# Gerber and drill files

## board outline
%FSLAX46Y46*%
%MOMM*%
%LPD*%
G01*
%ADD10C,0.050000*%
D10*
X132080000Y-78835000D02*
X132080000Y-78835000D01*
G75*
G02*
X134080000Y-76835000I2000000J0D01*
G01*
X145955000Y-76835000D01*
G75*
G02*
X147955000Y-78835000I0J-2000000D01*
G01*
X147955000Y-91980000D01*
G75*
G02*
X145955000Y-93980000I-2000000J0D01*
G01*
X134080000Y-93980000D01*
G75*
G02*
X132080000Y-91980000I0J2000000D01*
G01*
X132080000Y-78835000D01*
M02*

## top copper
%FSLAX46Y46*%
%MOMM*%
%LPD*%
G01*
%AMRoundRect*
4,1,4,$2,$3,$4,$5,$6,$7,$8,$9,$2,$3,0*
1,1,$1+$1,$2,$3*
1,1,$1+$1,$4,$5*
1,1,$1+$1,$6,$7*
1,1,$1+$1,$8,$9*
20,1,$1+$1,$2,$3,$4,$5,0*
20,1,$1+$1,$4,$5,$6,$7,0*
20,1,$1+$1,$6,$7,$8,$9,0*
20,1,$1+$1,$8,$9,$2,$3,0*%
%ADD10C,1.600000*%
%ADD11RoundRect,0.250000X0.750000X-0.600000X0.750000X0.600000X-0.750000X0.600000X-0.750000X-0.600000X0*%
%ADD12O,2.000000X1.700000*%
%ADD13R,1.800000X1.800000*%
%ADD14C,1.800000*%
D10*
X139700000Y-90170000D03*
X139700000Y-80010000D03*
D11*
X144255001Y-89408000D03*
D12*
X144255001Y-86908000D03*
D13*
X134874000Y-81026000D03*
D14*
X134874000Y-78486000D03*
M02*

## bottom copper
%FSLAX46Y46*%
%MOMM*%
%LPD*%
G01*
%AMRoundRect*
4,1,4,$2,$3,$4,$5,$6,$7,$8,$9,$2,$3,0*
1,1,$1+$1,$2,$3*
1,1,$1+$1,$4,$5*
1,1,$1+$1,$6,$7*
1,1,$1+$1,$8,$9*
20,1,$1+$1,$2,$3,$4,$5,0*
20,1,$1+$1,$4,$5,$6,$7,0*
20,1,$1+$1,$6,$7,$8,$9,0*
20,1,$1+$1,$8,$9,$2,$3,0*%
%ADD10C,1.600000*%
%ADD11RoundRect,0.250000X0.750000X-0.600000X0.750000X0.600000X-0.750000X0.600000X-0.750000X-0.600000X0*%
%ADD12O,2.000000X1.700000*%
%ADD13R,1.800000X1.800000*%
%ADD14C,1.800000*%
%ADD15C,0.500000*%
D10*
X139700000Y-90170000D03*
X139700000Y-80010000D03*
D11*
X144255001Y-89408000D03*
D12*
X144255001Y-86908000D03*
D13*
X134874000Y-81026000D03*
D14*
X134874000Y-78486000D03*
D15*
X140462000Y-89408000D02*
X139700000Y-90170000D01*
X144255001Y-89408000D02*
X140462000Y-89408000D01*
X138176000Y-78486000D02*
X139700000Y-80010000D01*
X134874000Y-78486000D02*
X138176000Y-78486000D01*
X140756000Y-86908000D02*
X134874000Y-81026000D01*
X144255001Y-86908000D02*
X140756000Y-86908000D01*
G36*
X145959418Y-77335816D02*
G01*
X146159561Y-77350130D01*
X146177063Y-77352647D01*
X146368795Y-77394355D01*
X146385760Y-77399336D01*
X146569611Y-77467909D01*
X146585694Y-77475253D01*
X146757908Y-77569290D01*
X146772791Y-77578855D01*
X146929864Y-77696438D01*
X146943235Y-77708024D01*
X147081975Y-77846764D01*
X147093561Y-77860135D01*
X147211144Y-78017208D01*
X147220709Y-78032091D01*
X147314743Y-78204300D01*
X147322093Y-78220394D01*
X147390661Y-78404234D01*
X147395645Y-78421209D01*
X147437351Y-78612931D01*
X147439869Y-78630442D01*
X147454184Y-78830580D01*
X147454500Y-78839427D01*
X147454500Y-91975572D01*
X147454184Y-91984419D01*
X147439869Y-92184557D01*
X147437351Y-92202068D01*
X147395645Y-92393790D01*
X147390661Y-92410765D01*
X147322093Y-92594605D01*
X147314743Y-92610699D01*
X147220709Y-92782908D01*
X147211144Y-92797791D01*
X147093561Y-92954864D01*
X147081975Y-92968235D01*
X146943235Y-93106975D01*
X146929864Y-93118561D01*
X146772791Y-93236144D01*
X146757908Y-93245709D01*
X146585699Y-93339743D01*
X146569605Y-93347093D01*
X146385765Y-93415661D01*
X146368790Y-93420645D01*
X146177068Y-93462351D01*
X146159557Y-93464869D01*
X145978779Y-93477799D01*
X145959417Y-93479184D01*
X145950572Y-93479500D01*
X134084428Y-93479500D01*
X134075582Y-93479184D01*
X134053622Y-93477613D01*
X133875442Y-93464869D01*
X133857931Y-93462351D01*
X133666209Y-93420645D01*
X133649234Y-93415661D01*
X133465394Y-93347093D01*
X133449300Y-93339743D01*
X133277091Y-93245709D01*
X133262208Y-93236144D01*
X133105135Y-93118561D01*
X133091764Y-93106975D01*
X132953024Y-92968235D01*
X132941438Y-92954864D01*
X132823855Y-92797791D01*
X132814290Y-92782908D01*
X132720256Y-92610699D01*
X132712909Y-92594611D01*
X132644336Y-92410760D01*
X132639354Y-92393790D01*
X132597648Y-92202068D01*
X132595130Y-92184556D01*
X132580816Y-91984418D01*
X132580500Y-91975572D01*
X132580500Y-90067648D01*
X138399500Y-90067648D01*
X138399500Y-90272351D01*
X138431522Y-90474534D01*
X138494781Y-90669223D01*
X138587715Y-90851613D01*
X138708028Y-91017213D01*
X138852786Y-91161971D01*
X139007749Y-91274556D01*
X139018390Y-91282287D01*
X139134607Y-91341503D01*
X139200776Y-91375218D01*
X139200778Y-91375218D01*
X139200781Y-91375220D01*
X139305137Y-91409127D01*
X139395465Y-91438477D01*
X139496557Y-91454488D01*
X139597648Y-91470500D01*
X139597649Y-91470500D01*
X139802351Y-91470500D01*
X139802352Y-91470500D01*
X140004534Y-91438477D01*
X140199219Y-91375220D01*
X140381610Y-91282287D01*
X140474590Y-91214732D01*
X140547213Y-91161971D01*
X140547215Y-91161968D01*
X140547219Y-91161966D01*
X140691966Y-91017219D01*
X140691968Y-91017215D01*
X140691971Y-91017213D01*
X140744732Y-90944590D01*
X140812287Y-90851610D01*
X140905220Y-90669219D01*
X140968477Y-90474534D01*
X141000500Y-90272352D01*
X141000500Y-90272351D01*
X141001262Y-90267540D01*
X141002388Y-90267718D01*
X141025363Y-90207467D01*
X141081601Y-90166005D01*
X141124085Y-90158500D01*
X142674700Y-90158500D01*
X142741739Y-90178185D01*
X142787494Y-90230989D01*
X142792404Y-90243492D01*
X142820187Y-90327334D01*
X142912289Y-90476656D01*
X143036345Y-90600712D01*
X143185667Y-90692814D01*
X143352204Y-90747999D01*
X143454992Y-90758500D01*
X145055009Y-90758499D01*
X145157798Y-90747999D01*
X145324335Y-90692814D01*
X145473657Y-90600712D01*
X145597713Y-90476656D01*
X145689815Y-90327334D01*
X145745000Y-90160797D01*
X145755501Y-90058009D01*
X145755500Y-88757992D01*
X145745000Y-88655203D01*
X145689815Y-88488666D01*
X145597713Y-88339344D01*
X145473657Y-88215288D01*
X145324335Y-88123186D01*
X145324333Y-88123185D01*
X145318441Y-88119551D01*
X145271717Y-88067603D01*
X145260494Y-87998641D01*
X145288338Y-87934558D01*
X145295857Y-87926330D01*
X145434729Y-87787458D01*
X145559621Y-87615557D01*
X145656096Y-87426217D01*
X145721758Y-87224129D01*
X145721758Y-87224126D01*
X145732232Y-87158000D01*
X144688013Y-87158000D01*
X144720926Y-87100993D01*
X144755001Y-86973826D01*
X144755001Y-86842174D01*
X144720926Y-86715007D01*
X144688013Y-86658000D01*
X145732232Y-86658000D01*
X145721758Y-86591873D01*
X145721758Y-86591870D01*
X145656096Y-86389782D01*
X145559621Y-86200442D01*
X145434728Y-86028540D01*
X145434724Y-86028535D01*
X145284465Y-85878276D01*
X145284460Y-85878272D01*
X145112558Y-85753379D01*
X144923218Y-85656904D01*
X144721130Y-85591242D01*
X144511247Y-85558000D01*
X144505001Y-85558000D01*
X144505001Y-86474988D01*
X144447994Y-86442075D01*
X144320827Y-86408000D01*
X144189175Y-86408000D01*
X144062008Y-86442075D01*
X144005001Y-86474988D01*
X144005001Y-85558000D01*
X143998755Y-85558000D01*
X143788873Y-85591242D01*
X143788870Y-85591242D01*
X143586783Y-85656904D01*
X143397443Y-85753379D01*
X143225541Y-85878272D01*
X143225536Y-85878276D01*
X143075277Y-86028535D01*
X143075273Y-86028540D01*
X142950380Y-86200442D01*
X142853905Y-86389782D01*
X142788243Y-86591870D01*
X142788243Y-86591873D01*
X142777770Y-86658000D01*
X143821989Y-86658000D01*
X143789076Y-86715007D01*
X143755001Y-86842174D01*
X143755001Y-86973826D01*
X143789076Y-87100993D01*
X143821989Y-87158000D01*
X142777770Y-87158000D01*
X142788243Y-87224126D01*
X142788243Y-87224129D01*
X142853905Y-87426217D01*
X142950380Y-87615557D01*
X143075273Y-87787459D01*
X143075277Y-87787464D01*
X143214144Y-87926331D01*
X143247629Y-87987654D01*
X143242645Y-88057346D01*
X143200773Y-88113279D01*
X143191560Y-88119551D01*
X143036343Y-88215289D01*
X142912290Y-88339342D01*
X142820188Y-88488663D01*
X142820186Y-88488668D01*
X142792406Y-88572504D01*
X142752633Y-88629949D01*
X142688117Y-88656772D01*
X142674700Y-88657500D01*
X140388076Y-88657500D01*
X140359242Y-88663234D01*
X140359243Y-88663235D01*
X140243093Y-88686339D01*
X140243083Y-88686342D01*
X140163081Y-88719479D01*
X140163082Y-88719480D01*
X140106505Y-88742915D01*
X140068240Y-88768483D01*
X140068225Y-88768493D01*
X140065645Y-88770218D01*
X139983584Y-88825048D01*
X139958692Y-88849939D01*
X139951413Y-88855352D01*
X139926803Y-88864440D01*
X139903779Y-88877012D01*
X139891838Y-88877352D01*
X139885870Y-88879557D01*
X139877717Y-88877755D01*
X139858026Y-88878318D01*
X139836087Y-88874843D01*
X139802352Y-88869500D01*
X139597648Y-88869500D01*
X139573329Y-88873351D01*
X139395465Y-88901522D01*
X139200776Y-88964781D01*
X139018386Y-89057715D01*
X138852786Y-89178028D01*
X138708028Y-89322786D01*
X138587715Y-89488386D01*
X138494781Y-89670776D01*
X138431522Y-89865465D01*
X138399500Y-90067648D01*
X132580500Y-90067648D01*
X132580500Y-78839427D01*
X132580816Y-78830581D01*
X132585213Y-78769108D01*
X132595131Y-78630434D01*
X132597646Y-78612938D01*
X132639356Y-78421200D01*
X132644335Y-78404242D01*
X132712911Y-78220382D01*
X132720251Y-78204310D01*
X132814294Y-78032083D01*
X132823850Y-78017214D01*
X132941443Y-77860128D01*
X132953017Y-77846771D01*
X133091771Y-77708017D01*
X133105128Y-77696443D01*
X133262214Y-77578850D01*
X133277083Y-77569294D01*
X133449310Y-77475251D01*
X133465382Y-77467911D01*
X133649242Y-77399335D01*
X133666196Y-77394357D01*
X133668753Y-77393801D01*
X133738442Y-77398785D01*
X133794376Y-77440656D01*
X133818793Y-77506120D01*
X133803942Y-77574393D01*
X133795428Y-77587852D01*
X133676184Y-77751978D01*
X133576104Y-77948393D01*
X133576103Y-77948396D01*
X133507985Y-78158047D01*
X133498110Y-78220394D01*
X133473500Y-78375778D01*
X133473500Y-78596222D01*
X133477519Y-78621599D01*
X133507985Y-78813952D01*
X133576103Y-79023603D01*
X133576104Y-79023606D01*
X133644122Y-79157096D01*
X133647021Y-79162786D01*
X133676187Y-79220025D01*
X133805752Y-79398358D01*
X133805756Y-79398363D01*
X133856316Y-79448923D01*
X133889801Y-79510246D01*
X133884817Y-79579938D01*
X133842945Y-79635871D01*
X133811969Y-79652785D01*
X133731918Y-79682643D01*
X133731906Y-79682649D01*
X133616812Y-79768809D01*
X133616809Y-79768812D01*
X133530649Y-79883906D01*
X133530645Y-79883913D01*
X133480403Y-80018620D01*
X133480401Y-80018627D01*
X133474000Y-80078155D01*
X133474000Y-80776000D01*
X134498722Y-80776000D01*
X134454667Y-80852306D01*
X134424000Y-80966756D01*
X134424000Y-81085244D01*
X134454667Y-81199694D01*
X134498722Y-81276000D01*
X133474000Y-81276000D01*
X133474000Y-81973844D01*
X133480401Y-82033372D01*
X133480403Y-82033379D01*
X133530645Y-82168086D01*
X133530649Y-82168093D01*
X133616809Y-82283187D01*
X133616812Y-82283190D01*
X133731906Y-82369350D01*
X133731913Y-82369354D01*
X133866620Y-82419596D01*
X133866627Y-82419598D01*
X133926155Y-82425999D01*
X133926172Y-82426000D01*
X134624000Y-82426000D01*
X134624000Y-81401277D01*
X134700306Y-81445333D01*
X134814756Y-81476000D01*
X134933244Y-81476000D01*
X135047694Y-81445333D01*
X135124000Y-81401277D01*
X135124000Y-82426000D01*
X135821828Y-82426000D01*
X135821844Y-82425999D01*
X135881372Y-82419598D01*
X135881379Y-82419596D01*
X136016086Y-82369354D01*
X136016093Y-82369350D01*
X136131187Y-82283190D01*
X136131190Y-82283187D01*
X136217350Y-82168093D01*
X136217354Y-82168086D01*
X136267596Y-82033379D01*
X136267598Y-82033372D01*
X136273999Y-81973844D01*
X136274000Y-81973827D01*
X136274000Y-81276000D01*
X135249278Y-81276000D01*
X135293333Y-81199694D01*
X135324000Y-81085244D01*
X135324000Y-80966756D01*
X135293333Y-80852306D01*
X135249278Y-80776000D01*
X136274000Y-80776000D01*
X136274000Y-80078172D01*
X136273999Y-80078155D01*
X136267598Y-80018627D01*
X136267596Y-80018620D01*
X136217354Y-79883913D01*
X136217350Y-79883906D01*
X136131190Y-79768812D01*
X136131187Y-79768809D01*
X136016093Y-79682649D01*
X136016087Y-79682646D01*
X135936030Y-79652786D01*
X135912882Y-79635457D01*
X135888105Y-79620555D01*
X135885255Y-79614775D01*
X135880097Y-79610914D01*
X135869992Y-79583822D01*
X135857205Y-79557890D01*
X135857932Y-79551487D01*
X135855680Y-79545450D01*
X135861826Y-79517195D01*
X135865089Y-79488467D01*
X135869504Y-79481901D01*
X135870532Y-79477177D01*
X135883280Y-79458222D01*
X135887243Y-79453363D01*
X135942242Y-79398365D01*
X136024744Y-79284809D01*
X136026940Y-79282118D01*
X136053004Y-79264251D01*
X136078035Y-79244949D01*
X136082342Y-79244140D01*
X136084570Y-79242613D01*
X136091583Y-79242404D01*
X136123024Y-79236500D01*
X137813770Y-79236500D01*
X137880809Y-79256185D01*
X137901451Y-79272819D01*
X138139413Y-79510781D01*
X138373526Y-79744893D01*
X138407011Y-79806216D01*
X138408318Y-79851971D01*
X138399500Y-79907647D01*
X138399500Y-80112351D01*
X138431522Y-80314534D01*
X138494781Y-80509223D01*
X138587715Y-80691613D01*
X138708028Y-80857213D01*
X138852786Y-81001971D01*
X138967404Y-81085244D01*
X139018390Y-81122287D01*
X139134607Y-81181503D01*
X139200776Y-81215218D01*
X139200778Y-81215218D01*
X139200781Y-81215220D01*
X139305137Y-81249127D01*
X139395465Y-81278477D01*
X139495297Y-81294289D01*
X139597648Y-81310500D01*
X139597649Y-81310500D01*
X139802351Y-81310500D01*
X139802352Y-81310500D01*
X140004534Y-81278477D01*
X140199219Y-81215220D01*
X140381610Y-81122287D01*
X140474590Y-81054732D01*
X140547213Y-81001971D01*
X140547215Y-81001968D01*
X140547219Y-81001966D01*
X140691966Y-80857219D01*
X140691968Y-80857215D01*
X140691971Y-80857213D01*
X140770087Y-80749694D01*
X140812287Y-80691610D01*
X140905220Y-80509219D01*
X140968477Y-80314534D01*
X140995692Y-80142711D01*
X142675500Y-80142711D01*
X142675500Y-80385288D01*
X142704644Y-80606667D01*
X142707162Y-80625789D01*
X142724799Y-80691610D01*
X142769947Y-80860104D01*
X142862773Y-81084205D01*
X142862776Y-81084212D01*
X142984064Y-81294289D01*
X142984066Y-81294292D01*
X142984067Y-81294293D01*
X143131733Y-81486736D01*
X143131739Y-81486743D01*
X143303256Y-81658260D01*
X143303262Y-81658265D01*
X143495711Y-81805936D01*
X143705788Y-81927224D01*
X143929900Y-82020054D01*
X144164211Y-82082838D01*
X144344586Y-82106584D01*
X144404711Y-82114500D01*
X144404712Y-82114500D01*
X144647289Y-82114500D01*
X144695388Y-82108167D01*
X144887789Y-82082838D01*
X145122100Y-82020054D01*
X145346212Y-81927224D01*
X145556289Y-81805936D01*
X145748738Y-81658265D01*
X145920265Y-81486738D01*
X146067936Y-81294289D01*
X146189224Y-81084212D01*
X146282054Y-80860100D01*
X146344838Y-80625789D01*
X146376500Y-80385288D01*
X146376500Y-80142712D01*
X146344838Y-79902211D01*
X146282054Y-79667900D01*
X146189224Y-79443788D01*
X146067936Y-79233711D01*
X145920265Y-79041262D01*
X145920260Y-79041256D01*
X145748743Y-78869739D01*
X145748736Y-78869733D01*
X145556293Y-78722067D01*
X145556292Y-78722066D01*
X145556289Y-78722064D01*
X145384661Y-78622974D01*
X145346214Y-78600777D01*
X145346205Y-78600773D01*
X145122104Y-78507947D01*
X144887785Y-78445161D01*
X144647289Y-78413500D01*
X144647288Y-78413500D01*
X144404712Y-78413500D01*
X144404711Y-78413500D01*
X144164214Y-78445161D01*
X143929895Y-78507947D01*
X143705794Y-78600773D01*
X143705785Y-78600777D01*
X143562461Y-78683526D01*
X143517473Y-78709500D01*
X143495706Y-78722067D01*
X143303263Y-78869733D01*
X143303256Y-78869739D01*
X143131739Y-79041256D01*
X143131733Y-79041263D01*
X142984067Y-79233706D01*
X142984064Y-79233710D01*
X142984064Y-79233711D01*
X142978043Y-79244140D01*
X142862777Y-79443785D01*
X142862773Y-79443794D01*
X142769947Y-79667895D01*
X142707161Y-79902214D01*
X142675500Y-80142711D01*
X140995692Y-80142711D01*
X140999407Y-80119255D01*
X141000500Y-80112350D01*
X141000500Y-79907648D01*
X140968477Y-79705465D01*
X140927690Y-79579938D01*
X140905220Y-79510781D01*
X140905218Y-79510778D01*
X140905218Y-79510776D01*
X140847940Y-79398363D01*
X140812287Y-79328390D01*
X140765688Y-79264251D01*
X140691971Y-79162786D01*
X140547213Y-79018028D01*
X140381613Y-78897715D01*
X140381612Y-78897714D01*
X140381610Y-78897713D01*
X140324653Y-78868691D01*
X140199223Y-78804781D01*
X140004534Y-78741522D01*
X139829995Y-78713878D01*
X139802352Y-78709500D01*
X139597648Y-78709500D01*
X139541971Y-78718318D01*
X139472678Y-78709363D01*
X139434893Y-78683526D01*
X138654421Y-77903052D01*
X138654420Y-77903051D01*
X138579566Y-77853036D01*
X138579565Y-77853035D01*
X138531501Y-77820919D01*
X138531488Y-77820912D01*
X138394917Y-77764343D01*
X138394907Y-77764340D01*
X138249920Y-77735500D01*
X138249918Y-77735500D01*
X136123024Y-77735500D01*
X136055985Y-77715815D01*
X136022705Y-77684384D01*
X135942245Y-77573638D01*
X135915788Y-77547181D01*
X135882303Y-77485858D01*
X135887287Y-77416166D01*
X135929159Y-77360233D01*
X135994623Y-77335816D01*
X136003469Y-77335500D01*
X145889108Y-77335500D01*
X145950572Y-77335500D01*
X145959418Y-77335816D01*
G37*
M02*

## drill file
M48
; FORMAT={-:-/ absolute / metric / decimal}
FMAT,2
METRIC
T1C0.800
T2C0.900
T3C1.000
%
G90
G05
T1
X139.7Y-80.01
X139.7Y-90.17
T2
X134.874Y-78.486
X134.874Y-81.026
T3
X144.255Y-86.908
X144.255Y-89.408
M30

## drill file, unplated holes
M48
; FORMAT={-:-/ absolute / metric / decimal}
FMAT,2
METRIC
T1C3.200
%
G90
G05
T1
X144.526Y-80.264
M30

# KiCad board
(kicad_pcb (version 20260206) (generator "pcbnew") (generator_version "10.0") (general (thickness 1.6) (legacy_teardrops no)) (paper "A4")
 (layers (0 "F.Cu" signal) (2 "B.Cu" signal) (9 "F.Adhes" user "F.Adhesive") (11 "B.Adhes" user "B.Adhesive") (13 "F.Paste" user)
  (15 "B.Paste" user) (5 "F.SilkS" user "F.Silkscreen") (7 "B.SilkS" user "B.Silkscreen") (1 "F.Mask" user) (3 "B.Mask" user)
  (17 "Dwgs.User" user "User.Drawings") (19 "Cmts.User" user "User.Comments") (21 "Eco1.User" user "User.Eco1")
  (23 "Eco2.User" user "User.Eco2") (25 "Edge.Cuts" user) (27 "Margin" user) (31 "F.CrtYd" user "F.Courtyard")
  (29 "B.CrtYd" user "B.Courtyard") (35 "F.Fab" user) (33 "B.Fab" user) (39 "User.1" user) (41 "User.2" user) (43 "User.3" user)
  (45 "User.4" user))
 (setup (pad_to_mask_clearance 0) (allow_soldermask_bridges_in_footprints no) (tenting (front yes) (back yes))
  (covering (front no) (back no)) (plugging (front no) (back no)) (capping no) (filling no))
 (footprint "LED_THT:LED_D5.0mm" (layer "F.Cu") (at 134.874 81.026 90)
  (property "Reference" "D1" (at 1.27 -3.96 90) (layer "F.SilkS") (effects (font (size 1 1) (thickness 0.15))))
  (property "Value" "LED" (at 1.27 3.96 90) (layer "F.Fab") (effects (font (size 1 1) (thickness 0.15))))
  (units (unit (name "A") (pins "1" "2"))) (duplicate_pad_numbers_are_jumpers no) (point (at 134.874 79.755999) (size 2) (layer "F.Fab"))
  (pad "1" thru_hole rect (at 0 0 90) (size 1.8 1.8) (drill 0.9) (layers "*.Cu" "*.Mask") (remove_unused_layers no) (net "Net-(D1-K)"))
  (pad "2" thru_hole circle (at 2.54 0 90) (size 1.8 1.8) (drill 0.9) (layers "*.Cu" "*.Mask") (remove_unused_layers no) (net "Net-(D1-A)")))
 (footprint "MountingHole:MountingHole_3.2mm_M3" (layer "F.Cu") (at 144.526 80.264)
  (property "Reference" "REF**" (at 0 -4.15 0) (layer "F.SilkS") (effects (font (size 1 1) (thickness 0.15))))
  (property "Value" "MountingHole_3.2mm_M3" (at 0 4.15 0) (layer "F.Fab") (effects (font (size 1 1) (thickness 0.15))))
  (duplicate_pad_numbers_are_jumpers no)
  (pad "" np_thru_hole circle (at 0 0) (size 3.2 3.2) (drill 3.2) (layers "*.Cu" "*.Mask")))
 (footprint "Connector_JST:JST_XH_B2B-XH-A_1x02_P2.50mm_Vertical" (layer "F.Cu") (at 144.255001 89.408 90)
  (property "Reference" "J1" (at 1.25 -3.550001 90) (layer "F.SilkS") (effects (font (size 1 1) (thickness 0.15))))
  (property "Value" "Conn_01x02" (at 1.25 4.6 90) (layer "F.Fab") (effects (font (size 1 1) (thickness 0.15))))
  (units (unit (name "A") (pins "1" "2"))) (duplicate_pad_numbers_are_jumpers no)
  (pad "1" thru_hole roundrect (at 0 0 90) (size 1.7 2) (drill 1) (layers "*.Cu" "*.Mask") (remove_unused_layers no)
   (roundrect_rratio 0.147059) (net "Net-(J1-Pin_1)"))
  (pad "2" thru_hole oval (at 2.5 0 90) (size 1.7 2) (drill 1) (layers "*.Cu" "*.Mask") (remove_unused_layers no) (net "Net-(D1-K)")))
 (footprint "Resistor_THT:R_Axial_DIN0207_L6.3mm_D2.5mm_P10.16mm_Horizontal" (layer "F.Cu") (at 139.7 80.01 -90)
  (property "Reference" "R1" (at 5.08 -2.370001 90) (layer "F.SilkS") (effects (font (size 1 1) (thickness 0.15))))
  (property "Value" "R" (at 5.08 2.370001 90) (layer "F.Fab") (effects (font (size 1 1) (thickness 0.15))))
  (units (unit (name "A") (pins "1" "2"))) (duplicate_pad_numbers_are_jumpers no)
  (pad "1" thru_hole circle (at 0 0 270) (size 1.6 1.6) (drill 0.8) (layers "*.Cu" "*.Mask") (remove_unused_layers no) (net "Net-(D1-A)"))
  (pad "2" thru_hole circle (at 10.16 0 270) (size 1.6 1.6) (drill 0.8) (layers "*.Cu" "*.Mask") (remove_unused_layers no)
   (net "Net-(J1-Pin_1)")))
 (gr_rect (start 132.08 76.835) (end 147.955 93.98) (radius 2) (stroke (width 0.05) (type solid)) (fill no) (layer "Edge.Cuts"))
 (segment (start 138.176 78.486) (end 139.7 80.01) (width 0.5) (layer "B.Cu") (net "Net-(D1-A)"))
 (segment (start 134.874 78.486) (end 138.176 78.486) (width 0.5) (layer "B.Cu") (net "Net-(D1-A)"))
 (segment (start 140.756 86.908) (end 134.874 81.026) (width 0.5) (layer "B.Cu") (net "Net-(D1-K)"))
 (segment (start 144.255001 86.908) (end 140.756 86.908) (width 0.5) (layer "B.Cu") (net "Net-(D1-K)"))
 (segment (start 140.462 89.408) (end 139.7 90.17) (width 0.5) (layer "B.Cu") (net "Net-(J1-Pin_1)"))
 (segment (start 144.255001 89.408) (end 140.462 89.408) (width 0.5) (layer "B.Cu") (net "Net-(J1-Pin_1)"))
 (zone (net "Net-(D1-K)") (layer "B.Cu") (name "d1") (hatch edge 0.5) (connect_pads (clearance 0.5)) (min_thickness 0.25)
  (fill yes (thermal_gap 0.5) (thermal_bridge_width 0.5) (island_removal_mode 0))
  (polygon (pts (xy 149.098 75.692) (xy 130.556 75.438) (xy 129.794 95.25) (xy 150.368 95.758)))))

